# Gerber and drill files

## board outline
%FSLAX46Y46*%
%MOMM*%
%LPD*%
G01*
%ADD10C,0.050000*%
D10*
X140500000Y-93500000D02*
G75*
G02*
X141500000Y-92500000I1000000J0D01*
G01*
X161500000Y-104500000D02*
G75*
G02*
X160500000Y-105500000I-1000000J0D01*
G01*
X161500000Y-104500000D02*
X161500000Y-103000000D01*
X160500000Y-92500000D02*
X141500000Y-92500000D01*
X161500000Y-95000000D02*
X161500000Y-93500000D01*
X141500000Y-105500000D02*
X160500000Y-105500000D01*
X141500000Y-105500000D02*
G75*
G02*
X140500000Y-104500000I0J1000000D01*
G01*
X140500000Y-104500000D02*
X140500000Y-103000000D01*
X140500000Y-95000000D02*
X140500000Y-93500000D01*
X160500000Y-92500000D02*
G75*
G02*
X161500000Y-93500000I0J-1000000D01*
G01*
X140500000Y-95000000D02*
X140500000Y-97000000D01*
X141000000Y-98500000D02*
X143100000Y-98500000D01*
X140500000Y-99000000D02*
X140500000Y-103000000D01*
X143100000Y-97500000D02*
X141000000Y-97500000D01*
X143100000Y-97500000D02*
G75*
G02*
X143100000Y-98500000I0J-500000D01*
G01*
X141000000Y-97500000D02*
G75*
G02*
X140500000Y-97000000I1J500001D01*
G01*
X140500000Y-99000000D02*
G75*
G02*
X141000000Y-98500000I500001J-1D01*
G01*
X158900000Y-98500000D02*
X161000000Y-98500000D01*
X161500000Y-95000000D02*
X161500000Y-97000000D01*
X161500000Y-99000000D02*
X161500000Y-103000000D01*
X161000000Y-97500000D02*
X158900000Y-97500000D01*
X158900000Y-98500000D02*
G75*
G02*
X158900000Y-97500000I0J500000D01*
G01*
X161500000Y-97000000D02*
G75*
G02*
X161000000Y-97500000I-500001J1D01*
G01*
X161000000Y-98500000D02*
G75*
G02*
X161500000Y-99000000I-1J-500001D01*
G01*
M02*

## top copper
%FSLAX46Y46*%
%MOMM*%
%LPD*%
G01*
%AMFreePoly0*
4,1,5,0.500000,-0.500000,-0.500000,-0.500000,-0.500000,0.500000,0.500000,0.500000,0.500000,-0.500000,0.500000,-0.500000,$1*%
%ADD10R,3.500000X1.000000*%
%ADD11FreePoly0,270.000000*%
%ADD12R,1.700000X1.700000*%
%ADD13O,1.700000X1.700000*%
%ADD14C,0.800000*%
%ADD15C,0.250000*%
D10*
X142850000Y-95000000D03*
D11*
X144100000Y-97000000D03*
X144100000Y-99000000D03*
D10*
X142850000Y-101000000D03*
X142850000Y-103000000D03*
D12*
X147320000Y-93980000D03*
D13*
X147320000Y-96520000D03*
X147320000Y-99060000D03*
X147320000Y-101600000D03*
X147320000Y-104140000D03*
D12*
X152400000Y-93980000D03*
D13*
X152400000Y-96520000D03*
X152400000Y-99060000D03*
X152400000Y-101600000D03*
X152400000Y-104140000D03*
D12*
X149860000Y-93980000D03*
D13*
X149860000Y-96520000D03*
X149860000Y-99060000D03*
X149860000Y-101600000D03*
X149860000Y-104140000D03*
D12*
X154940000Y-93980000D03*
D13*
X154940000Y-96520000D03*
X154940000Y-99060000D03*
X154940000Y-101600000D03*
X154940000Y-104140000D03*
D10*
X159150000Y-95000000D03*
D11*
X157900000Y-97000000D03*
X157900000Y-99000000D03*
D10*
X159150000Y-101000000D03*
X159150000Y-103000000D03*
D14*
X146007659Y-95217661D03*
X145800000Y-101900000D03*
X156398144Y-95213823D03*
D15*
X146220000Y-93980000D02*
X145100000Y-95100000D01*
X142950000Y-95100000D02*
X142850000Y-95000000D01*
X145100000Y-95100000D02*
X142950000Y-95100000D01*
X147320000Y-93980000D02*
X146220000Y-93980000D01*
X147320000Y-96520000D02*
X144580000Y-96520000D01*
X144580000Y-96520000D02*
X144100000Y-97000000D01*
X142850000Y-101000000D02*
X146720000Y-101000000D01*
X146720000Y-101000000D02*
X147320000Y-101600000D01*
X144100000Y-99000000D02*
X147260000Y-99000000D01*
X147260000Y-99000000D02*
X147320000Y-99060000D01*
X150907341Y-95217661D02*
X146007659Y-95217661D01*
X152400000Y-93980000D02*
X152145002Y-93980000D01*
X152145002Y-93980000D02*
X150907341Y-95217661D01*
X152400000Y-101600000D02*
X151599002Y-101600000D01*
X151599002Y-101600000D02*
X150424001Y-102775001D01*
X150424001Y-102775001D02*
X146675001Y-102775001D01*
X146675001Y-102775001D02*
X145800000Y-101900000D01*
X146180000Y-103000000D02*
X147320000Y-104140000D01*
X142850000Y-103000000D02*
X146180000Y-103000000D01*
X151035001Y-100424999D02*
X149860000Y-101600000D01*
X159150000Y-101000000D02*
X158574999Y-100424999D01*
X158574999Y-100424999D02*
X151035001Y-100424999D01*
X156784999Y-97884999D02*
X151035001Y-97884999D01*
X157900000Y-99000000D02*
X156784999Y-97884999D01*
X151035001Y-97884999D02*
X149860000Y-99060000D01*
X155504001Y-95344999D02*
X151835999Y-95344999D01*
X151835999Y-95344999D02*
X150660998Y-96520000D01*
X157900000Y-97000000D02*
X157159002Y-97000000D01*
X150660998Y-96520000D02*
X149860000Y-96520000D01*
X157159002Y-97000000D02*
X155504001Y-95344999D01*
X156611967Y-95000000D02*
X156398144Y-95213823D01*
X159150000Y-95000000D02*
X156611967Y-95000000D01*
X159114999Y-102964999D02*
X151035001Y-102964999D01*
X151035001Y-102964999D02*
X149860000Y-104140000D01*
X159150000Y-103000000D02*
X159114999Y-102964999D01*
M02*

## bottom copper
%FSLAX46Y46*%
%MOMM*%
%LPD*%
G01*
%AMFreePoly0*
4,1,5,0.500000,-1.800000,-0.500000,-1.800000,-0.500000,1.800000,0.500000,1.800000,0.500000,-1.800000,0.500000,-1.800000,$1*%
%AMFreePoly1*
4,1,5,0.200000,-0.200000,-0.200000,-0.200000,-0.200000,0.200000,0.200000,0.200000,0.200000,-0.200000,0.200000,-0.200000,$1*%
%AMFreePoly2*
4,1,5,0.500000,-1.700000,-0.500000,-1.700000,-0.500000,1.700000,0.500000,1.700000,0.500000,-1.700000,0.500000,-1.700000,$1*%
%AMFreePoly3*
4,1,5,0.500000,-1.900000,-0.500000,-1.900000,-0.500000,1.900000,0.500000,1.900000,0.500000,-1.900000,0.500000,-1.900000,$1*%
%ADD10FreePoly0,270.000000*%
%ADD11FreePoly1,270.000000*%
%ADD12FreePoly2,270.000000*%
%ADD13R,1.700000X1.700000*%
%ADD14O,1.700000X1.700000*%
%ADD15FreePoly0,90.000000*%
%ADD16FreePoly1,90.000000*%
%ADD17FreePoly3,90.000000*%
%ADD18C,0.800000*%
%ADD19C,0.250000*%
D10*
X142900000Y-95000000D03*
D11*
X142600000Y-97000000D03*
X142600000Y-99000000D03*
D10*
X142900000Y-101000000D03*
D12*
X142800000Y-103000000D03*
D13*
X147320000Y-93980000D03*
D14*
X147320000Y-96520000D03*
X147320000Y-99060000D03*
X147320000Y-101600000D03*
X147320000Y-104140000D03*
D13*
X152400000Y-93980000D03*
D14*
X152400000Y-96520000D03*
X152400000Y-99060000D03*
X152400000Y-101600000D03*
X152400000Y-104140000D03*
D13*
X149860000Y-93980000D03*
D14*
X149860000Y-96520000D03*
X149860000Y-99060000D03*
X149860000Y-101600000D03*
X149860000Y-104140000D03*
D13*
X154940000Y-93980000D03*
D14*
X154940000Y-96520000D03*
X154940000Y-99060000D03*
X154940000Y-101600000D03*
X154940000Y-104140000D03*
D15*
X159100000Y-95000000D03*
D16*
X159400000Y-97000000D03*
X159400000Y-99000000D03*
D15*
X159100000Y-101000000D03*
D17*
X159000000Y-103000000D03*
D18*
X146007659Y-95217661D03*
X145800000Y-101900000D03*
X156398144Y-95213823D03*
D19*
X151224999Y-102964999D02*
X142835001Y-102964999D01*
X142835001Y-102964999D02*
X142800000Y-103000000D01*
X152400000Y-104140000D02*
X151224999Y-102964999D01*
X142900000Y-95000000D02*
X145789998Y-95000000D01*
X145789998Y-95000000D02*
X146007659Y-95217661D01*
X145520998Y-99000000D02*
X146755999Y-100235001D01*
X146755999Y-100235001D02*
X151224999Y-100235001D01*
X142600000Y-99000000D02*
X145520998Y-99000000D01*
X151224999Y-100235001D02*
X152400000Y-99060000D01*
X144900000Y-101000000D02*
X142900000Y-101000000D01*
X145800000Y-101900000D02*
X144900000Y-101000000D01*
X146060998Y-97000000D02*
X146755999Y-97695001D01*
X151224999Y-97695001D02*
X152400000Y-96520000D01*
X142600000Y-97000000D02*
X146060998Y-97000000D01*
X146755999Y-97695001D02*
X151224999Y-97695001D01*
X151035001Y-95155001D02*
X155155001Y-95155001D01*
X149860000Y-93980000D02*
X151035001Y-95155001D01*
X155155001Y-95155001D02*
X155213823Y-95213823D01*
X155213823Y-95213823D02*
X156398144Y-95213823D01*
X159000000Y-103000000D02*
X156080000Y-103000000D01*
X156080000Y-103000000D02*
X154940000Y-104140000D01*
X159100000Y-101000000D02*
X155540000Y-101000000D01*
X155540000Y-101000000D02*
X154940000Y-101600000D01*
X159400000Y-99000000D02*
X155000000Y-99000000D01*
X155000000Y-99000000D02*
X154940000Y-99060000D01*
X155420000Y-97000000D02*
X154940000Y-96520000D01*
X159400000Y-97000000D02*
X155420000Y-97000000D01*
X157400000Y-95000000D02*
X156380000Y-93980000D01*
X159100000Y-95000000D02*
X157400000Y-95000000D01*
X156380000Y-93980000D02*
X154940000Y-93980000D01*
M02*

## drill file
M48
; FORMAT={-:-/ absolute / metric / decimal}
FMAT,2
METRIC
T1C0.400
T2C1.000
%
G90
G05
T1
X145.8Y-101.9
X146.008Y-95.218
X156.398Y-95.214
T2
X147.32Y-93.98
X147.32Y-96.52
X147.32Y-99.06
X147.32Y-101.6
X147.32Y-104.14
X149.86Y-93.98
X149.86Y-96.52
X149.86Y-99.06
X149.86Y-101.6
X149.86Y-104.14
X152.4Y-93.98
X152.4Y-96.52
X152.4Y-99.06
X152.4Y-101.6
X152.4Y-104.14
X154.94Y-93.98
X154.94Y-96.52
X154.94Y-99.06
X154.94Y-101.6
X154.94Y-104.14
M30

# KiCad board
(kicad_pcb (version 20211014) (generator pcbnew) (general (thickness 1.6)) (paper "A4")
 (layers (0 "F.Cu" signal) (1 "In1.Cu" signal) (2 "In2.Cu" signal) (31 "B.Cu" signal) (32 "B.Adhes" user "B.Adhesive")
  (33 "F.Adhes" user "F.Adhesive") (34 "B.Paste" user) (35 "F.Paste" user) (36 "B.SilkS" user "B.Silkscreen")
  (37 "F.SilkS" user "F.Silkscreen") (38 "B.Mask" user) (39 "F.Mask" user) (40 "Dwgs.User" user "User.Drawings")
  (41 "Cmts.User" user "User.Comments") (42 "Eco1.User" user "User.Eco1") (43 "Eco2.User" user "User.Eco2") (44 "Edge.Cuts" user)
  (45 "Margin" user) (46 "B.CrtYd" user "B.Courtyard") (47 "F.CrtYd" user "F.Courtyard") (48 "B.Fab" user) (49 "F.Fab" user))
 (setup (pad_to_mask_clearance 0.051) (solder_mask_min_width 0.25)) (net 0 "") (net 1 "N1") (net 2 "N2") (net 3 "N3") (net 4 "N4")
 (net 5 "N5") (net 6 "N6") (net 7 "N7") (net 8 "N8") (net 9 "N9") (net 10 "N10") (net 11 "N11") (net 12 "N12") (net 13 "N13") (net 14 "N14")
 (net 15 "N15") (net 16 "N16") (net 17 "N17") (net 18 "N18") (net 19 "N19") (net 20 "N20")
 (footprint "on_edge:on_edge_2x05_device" (layer "F.Cu") (at 140.5 99 -90)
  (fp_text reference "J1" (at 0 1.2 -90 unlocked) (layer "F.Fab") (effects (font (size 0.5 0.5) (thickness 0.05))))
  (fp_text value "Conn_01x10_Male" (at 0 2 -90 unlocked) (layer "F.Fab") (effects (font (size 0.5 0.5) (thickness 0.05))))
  (fp_line (start -4 0) (end -2 0) (layer "Edge.Cuts") (width 0.05))
  (fp_line (start -0.5 -0.5) (end -0.5 -2.6) (layer "Edge.Cuts") (width 0.05))
  (fp_line (start 0 0) (end 4 0) (layer "Edge.Cuts") (width 0.05))
  (fp_line (start -1.5 -2.6) (end -1.5 -0.5) (layer "Edge.Cuts") (width 0.05))
  (fp_arc (start -1.5 -2.6) (mid -1 -3.1) (end -0.5 -2.6) (layer "Edge.Cuts") (width 0.05))
  (fp_arc (start -1.5 -0.5) (mid -1.646447 -0.146447) (end -2 0) (layer "Edge.Cuts") (width 0.05))
  (fp_arc (start 0 0) (mid -0.353553 -0.146447) (end -0.5 -0.5) (layer "Edge.Cuts") (width 0.05))
  (pad "1" smd rect locked (at -4 -2.35 90) (size 1 3.5) (layers "F.Cu" "F.Mask") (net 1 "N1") (zone_connect 0))
  (pad "2" smd custom locked (at -2 -3.6 270) (size 1 1) (layers "F.Cu" "F.Mask") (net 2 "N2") (zone_connect 0)
   (options (clearance outline) (anchor rect)) (primitives))
  (pad "3" smd custom locked (at 0 -3.6 270) (size 1 1) (layers "F.Cu" "F.Mask") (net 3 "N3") (zone_connect 0)
   (options (clearance outline) (anchor rect)) (primitives))
  (pad "4" smd rect locked (at 2 -2.35 90) (size 1 3.5) (layers "F.Cu" "F.Mask") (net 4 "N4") (zone_connect 0))
  (pad "5" smd rect locked (at 4 -2.35 90) (size 1 3.5) (layers "F.Cu" "F.Mask") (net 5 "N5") (zone_connect 0))
  (pad "6" smd custom locked (at -4 -2.4 270) (size 1 3.6) (layers "B.Cu" "B.Mask") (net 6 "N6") (zone_connect 0)
   (options (clearance outline) (anchor rect)) (primitives))
  (pad "7" smd custom locked (at -2 -2.1 270) (size 0.4 0.4) (layers "B.Cu" "B.Mask") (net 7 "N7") (zone_connect 0)
   (options (clearance outline) (anchor rect)) (primitives))
  (pad "8" smd custom locked (at 0 -2.1 270) (size 0.4 0.4) (layers "B.Cu" "B.Mask") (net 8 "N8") (zone_connect 0)
   (options (clearance outline) (anchor rect)) (primitives))
  (pad "9" smd custom locked (at 2 -2.4 270) (size 1 3.6) (layers "B.Cu" "B.Mask") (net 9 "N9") (zone_connect 0)
   (options (clearance outline) (anchor rect)) (primitives))
  (pad "10" smd custom locked (at 4 -2.3 270) (size 1 3.4) (layers "B.Cu" "B.Mask") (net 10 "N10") (zone_connect 0)
   (options (clearance outline) (anchor rect)) (primitives)))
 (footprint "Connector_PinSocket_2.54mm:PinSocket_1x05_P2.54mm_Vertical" (layer "F.Cu") (at 147.32 93.98)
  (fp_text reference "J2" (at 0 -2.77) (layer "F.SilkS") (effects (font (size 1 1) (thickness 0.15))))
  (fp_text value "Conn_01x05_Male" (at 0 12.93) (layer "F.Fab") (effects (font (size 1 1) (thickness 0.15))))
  (pad "1" thru_hole rect locked (at 0 0) (size 1.7 1.7) (drill 1) (layers *.Cu *.Mask) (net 1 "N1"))
  (pad "2" thru_hole oval locked (at 0 2.54) (size 1.7 1.7) (drill 1) (layers *.Cu *.Mask) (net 2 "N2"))
  (pad "3" thru_hole oval locked (at 0 5.08) (size 1.7 1.7) (drill 1) (layers *.Cu *.Mask) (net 3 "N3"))
  (pad "4" thru_hole oval locked (at 0 7.62) (size 1.7 1.7) (drill 1) (layers *.Cu *.Mask) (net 4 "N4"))
  (pad "5" thru_hole oval locked (at 0 10.16) (size 1.7 1.7) (drill 1) (layers *.Cu *.Mask) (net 5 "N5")))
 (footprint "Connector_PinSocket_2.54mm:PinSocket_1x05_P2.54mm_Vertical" (layer "F.Cu") (at 152.4 93.98)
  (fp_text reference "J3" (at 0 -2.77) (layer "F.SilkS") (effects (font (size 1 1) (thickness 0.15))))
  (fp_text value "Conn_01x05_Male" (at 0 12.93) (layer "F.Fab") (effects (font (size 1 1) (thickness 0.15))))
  (pad "1" thru_hole rect locked (at 0 0) (size 1.7 1.7) (drill 1) (layers *.Cu *.Mask) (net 6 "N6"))
  (pad "2" thru_hole oval locked (at 0 2.54) (size 1.7 1.7) (drill 1) (layers *.Cu *.Mask) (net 7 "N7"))
  (pad "3" thru_hole oval locked (at 0 5.08) (size 1.7 1.7) (drill 1) (layers *.Cu *.Mask) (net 8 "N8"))
  (pad "4" thru_hole oval locked (at 0 7.62) (size 1.7 1.7) (drill 1) (layers *.Cu *.Mask) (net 9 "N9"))
  (pad "5" thru_hole oval locked (at 0 10.16) (size 1.7 1.7) (drill 1) (layers *.Cu *.Mask) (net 10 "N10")))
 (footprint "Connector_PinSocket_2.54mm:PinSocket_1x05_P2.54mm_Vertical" (layer "F.Cu") (at 149.86 93.98)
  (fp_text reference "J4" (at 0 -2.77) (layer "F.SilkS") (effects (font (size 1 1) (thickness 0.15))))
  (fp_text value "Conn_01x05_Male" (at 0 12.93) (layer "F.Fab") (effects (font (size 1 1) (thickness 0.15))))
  (pad "1" thru_hole rect locked (at 0 0) (size 1.7 1.7) (drill 1) (layers *.Cu *.Mask) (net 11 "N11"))
  (pad "2" thru_hole oval locked (at 0 2.54) (size 1.7 1.7) (drill 1) (layers *.Cu *.Mask) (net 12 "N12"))
  (pad "3" thru_hole oval locked (at 0 5.08) (size 1.7 1.7) (drill 1) (layers *.Cu *.Mask) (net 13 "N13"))
  (pad "4" thru_hole oval locked (at 0 7.62) (size 1.7 1.7) (drill 1) (layers *.Cu *.Mask) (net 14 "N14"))
  (pad "5" thru_hole oval locked (at 0 10.16) (size 1.7 1.7) (drill 1) (layers *.Cu *.Mask) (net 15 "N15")))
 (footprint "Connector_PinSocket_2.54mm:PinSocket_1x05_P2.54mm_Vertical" (layer "F.Cu") (at 154.94 93.98)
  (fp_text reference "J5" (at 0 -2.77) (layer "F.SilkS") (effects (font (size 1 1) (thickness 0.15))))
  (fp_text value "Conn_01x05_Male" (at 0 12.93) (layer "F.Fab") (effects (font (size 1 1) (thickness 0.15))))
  (pad "1" thru_hole rect locked (at 0 0) (size 1.7 1.7) (drill 1) (layers *.Cu *.Mask) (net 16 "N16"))
  (pad "2" thru_hole oval locked (at 0 2.54) (size 1.7 1.7) (drill 1) (layers *.Cu *.Mask) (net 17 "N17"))
  (pad "3" thru_hole oval locked (at 0 5.08) (size 1.7 1.7) (drill 1) (layers *.Cu *.Mask) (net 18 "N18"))
  (pad "4" thru_hole oval locked (at 0 7.62) (size 1.7 1.7) (drill 1) (layers *.Cu *.Mask) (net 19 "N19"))
  (pad "5" thru_hole oval locked (at 0 10.16) (size 1.7 1.7) (drill 1) (layers *.Cu *.Mask) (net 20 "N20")))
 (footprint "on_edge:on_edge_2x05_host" (layer "F.Cu") (at 161.5 99 -90)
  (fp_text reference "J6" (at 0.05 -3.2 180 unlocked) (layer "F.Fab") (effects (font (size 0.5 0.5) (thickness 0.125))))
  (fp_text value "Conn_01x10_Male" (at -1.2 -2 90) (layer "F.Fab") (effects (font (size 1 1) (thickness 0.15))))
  (fp_line (start -0.5 2.6) (end -0.5 0.5) (layer "Edge.Cuts") (width 0.05))
  (fp_line (start -4 0) (end -2 0) (layer "Edge.Cuts") (width 0.05))
  (fp_line (start 0 0) (end 4 0) (layer "Edge.Cuts") (width 0.05))
  (fp_line (start -1.5 0.5) (end -1.5 2.6) (layer "Edge.Cuts") (width 0.05))
  (fp_arc (start -0.5 2.6) (mid -1 3.1) (end -1.5 2.6) (layer "Edge.Cuts") (width 0.05))
  (fp_arc (start -2 0) (mid -1.646447 0.146447) (end -1.5 0.5) (layer "Edge.Cuts") (width 0.05))
  (fp_arc (start -0.5 0.5) (mid -0.353553 0.146447) (end 0 0) (layer "Edge.Cuts") (width 0.05))
  (pad "1" smd rect locked (at -4 2.35 270) (size 1 3.5) (layers "F.Cu" "F.Mask") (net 11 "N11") (zone_connect 0))
  (pad "2" smd custom locked (at -2 3.6 270) (size 1 1) (layers "F.Cu" "F.Mask") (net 12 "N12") (zone_connect 0)
   (options (clearance outline) (anchor rect)) (primitives))
  (pad "3" smd custom locked (at 0 3.6 270) (size 1 1) (layers "F.Cu" "F.Mask") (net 13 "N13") (zone_connect 0)
   (options (clearance outline) (anchor rect)) (primitives))
  (pad "4" smd rect locked (at 2 2.35 270) (size 1 3.5) (layers "F.Cu" "F.Mask") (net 14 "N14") (zone_connect 0))
  (pad "5" smd rect locked (at 4 2.35 270) (size 1 3.5) (layers "F.Cu" "F.Mask") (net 15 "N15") (zone_connect 0))
  (pad "6" smd custom locked (at -4 2.4 90) (size 1 3.6) (layers "B.Cu" "B.Mask") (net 16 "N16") (zone_connect 0)
   (options (clearance outline) (anchor rect)) (primitives))
  (pad "7" smd custom locked (at -2 2.1 90) (size 0.4 0.4) (layers "B.Cu" "B.Mask") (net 17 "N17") (zone_connect 0)
   (options (clearance outline) (anchor rect)) (primitives))
  (pad "8" smd custom locked (at 0 2.1 90) (size 0.4 0.4) (layers "B.Cu" "B.Mask") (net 18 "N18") (zone_connect 0)
   (options (clearance outline) (anchor rect)) (primitives))
  (pad "9" smd custom locked (at 2 2.4 90) (size 1 3.6) (layers "B.Cu" "B.Mask") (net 19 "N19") (zone_connect 0)
   (options (clearance outline) (anchor rect)) (primitives))
  (pad "10" smd custom locked (at 4 2.5 90) (size 1 3.8) (layers "B.Cu" "B.Mask") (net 20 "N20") (zone_connect 0)
   (options (clearance outline) (anchor rect)) (primitives)))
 (gr_arc (start 140.5 93.5) (mid 140.792893 92.792893) (end 141.5 92.5) (layer "Edge.Cuts") (width 0.05))
 (gr_arc (start 161.5 104.5) (mid 161.207107 105.207107) (end 160.5 105.5) (layer "Edge.Cuts") (width 0.05))
 (gr_line (start 161.5 104.5) (end 161.5 103) (layer "Edge.Cuts") (width 0.05))
 (gr_line (start 160.5 92.5) (end 141.5 92.5) (layer "Edge.Cuts") (width 0.05))
 (gr_line (start 161.5 95) (end 161.5 93.5) (layer "Edge.Cuts") (width 0.05))
 (gr_line (start 141.5 105.5) (end 160.5 105.5) (layer "Edge.Cuts") (width 0.05))
 (gr_arc (start 141.5 105.5) (mid 140.792893 105.207107) (end 140.5 104.5) (layer "Edge.Cuts") (width 0.05))
 (gr_line (start 140.5 104.5) (end 140.5 103) (layer "Edge.Cuts") (width 0.05))
 (gr_line (start 140.5 95) (end 140.5 93.5) (layer "Edge.Cuts") (width 0.05))
 (gr_arc (start 160.5 92.5) (mid 161.207107 92.792893) (end 161.5 93.5) (layer "Edge.Cuts") (width 0.05))
 (segment (start 146.22 93.98) (end 145.1 95.1) (width 0.25) (layer "F.Cu") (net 1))
 (segment (start 142.95 95.1) (end 142.85 95) (width 0.25) (layer "F.Cu") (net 1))
 (segment (start 145.1 95.1) (end 142.95 95.1) (width 0.25) (layer "F.Cu") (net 1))
 (segment (start 147.32 93.98) (end 146.22 93.98) (width 0.25) (layer "F.Cu") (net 1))
 (segment (start 147.32 96.52) (end 144.58 96.52) (width 0.25) (layer "F.Cu") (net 2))
 (segment (start 144.58 96.52) (end 144.1 97) (width 0.25) (layer "F.Cu") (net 2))
 (segment (start 142.85 101) (end 146.72 101) (width 0.25) (layer "F.Cu") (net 4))
 (segment (start 146.72 101) (end 147.32 101.6) (width 0.25) (layer "F.Cu") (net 4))
 (segment (start 144.1 99) (end 147.26 99) (width 0.25) (layer "F.Cu") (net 3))
 (segment (start 147.26 99) (end 147.32 99.06) (width 0.25) (layer "F.Cu") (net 3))
 (segment (start 151.224999 102.964999) (end 142.835001 102.964999) (width 0.25) (layer "B.Cu") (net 10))
 (segment (start 142.835001 102.964999) (end 142.8 103) (width 0.25) (layer "B.Cu") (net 10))
 (segment (start 152.4 104.14) (end 151.224999 102.964999) (width 0.25) (layer "B.Cu") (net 10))
 (segment (start 150.907341 95.217661) (end 146.007659 95.217661) (width 0.25) (layer "F.Cu") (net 6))
 (segment (start 152.4 93.98) (end 152.145002 93.98) (width 0.25) (layer "F.Cu") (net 6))
 (segment (start 152.145002 93.98) (end 150.907341 95.217661) (width 0.25) (layer "F.Cu") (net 6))
 (via (at 146.007659 95.217661) (size 0.8) (drill 0.4) (layers "F.Cu" "B.Cu") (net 6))
 (segment (start 142.9 95) (end 145.789998 95) (width 0.25) (layer "B.Cu") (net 6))
 (segment (start 145.789998 95) (end 146.007659 95.217661) (width 0.25) (layer "B.Cu") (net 6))
 (segment (start 145.520998 99) (end 146.755999 100.235001) (width 0.25) (layer "B.Cu") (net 8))
 (segment (start 146.755999 100.235001) (end 151.224999 100.235001) (width 0.25) (layer "B.Cu") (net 8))
 (segment (start 142.6 99) (end 145.520998 99) (width 0.25) (layer "B.Cu") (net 8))
 (segment (start 151.224999 100.235001) (end 152.4 99.06) (width 0.25) (layer "B.Cu") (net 8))
 (segment (start 152.4 101.6) (end 151.599002 101.6) (width 0.25) (layer "F.Cu") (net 9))
 (segment (start 151.599002 101.6) (end 150.424001 102.775001) (width 0.25) (layer "F.Cu") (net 9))
 (segment (start 150.424001 102.775001) (end 146.675001 102.775001) (width 0.25) (layer "F.Cu") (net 9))
 (segment (start 146.675001 102.775001) (end 145.8 101.9) (width 0.25) (layer "F.Cu") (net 9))
 (via (at 145.8 101.9) (size 0.8) (drill 0.4) (layers "F.Cu" "B.Cu") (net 9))
 (segment (start 144.9 101) (end 142.9 101) (width 0.25) (layer "B.Cu") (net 9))
 (segment (start 145.8 101.9) (end 144.9 101) (width 0.25) (layer "B.Cu") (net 9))
 (segment (start 146.060998 97) (end 146.755999 97.695001) (width 0.25) (layer "B.Cu") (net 7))
 (segment (start 151.224999 97.695001) (end 152.4 96.52) (width 0.25) (layer "B.Cu") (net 7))
 (segment (start 142.6 97) (end 146.060998 97) (width 0.25) (layer "B.Cu") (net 7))
 (segment (start 146.755999 97.695001) (end 151.224999 97.695001) (width 0.25) (layer "B.Cu") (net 7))
 (segment (start 146.18 103) (end 147.32 104.14) (width 0.25) (layer "F.Cu") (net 5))
 (segment (start 142.85 103) (end 146.18 103) (width 0.25) (layer "F.Cu") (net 5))
 (segment (start 151.035001 100.424999) (end 149.86 101.6) (width 0.25) (layer "F.Cu") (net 14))
 (segment (start 159.15 101) (end 158.574999 100.424999) (width 0.25) (layer "F.Cu") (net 14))
 (segment (start 158.574999 100.424999) (end 151.035001 100.424999) (width 0.25) (layer "F.Cu") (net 14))
 (segment (start 156.784999 97.884999) (end 151.035001 97.884999) (width 0.25) (layer "F.Cu") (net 13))
 (segment (start 157.9 99) (end 156.784999 97.884999) (width 0.25) (layer "F.Cu") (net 13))
 (segment (start 151.035001 97.884999) (end 149.86 99.06) (width 0.25) (layer "F.Cu") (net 13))
 (segment (start 155.504001 95.344999) (end 151.835999 95.344999) (width 0.25) (layer "F.Cu") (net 12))
 (segment (start 151.835999 95.344999) (end 150.660998 96.52) (width 0.25) (layer "F.Cu") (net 12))
 (segment (start 157.9 97) (end 157.159002 97) (width 0.25) (layer "F.Cu") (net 12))
 (segment (start 150.660998 96.52) (end 149.86 96.52) (width 0.25) (layer "F.Cu") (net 12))
 (segment (start 157.159002 97) (end 155.504001 95.344999) (width 0.25) (layer "F.Cu") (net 12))
 (segment (start 156.611967 95) (end 156.398144 95.213823) (width 0.25) (layer "F.Cu") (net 11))
 (segment (start 159.15 95) (end 156.611967 95) (width 0.25) (layer "F.Cu") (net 11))
 (via (at 156.398144 95.213823) (size 0.8) (drill 0.4) (layers "F.Cu" "B.Cu") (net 11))
 (segment (start 151.035001 95.155001) (end 155.155001 95.155001) (width 0.25) (layer "B.Cu") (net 11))
 (segment (start 149.86 93.98) (end 151.035001 95.155001) (width 0.25) (layer "B.Cu") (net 11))
 (segment (start 155.155001 95.155001) (end 155.213823 95.213823) (width 0.25) (layer "B.Cu") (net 11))
 (segment (start 155.213823 95.213823) (end 156.398144 95.213823) (width 0.25) (layer "B.Cu") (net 11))
 (segment (start 159.114999 102.964999) (end 151.035001 102.964999) (width 0.25) (layer "F.Cu") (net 15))
 (segment (start 151.035001 102.964999) (end 149.86 104.14) (width 0.25) (layer "F.Cu") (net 15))
 (segment (start 159.15 103) (end 159.114999 102.964999) (width 0.25) (layer "F.Cu") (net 15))
 (segment (start 159 103) (end 156.08 103) (width 0.25) (layer "B.Cu") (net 20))
 (segment (start 156.08 103) (end 154.94 104.14) (width 0.25) (layer "B.Cu") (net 20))
 (segment (start 159.1 101) (end 155.54 101) (width 0.25) (layer "B.Cu") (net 19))
 (segment (start 155.54 101) (end 154.94 101.6) (width 0.25) (layer "B.Cu") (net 19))
 (segment (start 159.4 99) (end 155 99) (width 0.25) (layer "B.Cu") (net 18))
 (segment (start 155 99) (end 154.94 99.06) (width 0.25) (layer "B.Cu") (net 18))
 (segment (start 155.42 97) (end 154.94 96.52) (width 0.25) (layer "B.Cu") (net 17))
 (segment (start 159.4 97) (end 155.42 97) (width 0.25) (layer "B.Cu") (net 17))
 (segment (start 157.4 95) (end 156.38 93.98) (width 0.25) (layer "B.Cu") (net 16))
 (segment (start 159.1 95) (end 157.4 95) (width 0.25) (layer "B.Cu") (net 16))
 (segment (start 156.38 93.98) (end 154.94 93.98) (width 0.25) (layer "B.Cu") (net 16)))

